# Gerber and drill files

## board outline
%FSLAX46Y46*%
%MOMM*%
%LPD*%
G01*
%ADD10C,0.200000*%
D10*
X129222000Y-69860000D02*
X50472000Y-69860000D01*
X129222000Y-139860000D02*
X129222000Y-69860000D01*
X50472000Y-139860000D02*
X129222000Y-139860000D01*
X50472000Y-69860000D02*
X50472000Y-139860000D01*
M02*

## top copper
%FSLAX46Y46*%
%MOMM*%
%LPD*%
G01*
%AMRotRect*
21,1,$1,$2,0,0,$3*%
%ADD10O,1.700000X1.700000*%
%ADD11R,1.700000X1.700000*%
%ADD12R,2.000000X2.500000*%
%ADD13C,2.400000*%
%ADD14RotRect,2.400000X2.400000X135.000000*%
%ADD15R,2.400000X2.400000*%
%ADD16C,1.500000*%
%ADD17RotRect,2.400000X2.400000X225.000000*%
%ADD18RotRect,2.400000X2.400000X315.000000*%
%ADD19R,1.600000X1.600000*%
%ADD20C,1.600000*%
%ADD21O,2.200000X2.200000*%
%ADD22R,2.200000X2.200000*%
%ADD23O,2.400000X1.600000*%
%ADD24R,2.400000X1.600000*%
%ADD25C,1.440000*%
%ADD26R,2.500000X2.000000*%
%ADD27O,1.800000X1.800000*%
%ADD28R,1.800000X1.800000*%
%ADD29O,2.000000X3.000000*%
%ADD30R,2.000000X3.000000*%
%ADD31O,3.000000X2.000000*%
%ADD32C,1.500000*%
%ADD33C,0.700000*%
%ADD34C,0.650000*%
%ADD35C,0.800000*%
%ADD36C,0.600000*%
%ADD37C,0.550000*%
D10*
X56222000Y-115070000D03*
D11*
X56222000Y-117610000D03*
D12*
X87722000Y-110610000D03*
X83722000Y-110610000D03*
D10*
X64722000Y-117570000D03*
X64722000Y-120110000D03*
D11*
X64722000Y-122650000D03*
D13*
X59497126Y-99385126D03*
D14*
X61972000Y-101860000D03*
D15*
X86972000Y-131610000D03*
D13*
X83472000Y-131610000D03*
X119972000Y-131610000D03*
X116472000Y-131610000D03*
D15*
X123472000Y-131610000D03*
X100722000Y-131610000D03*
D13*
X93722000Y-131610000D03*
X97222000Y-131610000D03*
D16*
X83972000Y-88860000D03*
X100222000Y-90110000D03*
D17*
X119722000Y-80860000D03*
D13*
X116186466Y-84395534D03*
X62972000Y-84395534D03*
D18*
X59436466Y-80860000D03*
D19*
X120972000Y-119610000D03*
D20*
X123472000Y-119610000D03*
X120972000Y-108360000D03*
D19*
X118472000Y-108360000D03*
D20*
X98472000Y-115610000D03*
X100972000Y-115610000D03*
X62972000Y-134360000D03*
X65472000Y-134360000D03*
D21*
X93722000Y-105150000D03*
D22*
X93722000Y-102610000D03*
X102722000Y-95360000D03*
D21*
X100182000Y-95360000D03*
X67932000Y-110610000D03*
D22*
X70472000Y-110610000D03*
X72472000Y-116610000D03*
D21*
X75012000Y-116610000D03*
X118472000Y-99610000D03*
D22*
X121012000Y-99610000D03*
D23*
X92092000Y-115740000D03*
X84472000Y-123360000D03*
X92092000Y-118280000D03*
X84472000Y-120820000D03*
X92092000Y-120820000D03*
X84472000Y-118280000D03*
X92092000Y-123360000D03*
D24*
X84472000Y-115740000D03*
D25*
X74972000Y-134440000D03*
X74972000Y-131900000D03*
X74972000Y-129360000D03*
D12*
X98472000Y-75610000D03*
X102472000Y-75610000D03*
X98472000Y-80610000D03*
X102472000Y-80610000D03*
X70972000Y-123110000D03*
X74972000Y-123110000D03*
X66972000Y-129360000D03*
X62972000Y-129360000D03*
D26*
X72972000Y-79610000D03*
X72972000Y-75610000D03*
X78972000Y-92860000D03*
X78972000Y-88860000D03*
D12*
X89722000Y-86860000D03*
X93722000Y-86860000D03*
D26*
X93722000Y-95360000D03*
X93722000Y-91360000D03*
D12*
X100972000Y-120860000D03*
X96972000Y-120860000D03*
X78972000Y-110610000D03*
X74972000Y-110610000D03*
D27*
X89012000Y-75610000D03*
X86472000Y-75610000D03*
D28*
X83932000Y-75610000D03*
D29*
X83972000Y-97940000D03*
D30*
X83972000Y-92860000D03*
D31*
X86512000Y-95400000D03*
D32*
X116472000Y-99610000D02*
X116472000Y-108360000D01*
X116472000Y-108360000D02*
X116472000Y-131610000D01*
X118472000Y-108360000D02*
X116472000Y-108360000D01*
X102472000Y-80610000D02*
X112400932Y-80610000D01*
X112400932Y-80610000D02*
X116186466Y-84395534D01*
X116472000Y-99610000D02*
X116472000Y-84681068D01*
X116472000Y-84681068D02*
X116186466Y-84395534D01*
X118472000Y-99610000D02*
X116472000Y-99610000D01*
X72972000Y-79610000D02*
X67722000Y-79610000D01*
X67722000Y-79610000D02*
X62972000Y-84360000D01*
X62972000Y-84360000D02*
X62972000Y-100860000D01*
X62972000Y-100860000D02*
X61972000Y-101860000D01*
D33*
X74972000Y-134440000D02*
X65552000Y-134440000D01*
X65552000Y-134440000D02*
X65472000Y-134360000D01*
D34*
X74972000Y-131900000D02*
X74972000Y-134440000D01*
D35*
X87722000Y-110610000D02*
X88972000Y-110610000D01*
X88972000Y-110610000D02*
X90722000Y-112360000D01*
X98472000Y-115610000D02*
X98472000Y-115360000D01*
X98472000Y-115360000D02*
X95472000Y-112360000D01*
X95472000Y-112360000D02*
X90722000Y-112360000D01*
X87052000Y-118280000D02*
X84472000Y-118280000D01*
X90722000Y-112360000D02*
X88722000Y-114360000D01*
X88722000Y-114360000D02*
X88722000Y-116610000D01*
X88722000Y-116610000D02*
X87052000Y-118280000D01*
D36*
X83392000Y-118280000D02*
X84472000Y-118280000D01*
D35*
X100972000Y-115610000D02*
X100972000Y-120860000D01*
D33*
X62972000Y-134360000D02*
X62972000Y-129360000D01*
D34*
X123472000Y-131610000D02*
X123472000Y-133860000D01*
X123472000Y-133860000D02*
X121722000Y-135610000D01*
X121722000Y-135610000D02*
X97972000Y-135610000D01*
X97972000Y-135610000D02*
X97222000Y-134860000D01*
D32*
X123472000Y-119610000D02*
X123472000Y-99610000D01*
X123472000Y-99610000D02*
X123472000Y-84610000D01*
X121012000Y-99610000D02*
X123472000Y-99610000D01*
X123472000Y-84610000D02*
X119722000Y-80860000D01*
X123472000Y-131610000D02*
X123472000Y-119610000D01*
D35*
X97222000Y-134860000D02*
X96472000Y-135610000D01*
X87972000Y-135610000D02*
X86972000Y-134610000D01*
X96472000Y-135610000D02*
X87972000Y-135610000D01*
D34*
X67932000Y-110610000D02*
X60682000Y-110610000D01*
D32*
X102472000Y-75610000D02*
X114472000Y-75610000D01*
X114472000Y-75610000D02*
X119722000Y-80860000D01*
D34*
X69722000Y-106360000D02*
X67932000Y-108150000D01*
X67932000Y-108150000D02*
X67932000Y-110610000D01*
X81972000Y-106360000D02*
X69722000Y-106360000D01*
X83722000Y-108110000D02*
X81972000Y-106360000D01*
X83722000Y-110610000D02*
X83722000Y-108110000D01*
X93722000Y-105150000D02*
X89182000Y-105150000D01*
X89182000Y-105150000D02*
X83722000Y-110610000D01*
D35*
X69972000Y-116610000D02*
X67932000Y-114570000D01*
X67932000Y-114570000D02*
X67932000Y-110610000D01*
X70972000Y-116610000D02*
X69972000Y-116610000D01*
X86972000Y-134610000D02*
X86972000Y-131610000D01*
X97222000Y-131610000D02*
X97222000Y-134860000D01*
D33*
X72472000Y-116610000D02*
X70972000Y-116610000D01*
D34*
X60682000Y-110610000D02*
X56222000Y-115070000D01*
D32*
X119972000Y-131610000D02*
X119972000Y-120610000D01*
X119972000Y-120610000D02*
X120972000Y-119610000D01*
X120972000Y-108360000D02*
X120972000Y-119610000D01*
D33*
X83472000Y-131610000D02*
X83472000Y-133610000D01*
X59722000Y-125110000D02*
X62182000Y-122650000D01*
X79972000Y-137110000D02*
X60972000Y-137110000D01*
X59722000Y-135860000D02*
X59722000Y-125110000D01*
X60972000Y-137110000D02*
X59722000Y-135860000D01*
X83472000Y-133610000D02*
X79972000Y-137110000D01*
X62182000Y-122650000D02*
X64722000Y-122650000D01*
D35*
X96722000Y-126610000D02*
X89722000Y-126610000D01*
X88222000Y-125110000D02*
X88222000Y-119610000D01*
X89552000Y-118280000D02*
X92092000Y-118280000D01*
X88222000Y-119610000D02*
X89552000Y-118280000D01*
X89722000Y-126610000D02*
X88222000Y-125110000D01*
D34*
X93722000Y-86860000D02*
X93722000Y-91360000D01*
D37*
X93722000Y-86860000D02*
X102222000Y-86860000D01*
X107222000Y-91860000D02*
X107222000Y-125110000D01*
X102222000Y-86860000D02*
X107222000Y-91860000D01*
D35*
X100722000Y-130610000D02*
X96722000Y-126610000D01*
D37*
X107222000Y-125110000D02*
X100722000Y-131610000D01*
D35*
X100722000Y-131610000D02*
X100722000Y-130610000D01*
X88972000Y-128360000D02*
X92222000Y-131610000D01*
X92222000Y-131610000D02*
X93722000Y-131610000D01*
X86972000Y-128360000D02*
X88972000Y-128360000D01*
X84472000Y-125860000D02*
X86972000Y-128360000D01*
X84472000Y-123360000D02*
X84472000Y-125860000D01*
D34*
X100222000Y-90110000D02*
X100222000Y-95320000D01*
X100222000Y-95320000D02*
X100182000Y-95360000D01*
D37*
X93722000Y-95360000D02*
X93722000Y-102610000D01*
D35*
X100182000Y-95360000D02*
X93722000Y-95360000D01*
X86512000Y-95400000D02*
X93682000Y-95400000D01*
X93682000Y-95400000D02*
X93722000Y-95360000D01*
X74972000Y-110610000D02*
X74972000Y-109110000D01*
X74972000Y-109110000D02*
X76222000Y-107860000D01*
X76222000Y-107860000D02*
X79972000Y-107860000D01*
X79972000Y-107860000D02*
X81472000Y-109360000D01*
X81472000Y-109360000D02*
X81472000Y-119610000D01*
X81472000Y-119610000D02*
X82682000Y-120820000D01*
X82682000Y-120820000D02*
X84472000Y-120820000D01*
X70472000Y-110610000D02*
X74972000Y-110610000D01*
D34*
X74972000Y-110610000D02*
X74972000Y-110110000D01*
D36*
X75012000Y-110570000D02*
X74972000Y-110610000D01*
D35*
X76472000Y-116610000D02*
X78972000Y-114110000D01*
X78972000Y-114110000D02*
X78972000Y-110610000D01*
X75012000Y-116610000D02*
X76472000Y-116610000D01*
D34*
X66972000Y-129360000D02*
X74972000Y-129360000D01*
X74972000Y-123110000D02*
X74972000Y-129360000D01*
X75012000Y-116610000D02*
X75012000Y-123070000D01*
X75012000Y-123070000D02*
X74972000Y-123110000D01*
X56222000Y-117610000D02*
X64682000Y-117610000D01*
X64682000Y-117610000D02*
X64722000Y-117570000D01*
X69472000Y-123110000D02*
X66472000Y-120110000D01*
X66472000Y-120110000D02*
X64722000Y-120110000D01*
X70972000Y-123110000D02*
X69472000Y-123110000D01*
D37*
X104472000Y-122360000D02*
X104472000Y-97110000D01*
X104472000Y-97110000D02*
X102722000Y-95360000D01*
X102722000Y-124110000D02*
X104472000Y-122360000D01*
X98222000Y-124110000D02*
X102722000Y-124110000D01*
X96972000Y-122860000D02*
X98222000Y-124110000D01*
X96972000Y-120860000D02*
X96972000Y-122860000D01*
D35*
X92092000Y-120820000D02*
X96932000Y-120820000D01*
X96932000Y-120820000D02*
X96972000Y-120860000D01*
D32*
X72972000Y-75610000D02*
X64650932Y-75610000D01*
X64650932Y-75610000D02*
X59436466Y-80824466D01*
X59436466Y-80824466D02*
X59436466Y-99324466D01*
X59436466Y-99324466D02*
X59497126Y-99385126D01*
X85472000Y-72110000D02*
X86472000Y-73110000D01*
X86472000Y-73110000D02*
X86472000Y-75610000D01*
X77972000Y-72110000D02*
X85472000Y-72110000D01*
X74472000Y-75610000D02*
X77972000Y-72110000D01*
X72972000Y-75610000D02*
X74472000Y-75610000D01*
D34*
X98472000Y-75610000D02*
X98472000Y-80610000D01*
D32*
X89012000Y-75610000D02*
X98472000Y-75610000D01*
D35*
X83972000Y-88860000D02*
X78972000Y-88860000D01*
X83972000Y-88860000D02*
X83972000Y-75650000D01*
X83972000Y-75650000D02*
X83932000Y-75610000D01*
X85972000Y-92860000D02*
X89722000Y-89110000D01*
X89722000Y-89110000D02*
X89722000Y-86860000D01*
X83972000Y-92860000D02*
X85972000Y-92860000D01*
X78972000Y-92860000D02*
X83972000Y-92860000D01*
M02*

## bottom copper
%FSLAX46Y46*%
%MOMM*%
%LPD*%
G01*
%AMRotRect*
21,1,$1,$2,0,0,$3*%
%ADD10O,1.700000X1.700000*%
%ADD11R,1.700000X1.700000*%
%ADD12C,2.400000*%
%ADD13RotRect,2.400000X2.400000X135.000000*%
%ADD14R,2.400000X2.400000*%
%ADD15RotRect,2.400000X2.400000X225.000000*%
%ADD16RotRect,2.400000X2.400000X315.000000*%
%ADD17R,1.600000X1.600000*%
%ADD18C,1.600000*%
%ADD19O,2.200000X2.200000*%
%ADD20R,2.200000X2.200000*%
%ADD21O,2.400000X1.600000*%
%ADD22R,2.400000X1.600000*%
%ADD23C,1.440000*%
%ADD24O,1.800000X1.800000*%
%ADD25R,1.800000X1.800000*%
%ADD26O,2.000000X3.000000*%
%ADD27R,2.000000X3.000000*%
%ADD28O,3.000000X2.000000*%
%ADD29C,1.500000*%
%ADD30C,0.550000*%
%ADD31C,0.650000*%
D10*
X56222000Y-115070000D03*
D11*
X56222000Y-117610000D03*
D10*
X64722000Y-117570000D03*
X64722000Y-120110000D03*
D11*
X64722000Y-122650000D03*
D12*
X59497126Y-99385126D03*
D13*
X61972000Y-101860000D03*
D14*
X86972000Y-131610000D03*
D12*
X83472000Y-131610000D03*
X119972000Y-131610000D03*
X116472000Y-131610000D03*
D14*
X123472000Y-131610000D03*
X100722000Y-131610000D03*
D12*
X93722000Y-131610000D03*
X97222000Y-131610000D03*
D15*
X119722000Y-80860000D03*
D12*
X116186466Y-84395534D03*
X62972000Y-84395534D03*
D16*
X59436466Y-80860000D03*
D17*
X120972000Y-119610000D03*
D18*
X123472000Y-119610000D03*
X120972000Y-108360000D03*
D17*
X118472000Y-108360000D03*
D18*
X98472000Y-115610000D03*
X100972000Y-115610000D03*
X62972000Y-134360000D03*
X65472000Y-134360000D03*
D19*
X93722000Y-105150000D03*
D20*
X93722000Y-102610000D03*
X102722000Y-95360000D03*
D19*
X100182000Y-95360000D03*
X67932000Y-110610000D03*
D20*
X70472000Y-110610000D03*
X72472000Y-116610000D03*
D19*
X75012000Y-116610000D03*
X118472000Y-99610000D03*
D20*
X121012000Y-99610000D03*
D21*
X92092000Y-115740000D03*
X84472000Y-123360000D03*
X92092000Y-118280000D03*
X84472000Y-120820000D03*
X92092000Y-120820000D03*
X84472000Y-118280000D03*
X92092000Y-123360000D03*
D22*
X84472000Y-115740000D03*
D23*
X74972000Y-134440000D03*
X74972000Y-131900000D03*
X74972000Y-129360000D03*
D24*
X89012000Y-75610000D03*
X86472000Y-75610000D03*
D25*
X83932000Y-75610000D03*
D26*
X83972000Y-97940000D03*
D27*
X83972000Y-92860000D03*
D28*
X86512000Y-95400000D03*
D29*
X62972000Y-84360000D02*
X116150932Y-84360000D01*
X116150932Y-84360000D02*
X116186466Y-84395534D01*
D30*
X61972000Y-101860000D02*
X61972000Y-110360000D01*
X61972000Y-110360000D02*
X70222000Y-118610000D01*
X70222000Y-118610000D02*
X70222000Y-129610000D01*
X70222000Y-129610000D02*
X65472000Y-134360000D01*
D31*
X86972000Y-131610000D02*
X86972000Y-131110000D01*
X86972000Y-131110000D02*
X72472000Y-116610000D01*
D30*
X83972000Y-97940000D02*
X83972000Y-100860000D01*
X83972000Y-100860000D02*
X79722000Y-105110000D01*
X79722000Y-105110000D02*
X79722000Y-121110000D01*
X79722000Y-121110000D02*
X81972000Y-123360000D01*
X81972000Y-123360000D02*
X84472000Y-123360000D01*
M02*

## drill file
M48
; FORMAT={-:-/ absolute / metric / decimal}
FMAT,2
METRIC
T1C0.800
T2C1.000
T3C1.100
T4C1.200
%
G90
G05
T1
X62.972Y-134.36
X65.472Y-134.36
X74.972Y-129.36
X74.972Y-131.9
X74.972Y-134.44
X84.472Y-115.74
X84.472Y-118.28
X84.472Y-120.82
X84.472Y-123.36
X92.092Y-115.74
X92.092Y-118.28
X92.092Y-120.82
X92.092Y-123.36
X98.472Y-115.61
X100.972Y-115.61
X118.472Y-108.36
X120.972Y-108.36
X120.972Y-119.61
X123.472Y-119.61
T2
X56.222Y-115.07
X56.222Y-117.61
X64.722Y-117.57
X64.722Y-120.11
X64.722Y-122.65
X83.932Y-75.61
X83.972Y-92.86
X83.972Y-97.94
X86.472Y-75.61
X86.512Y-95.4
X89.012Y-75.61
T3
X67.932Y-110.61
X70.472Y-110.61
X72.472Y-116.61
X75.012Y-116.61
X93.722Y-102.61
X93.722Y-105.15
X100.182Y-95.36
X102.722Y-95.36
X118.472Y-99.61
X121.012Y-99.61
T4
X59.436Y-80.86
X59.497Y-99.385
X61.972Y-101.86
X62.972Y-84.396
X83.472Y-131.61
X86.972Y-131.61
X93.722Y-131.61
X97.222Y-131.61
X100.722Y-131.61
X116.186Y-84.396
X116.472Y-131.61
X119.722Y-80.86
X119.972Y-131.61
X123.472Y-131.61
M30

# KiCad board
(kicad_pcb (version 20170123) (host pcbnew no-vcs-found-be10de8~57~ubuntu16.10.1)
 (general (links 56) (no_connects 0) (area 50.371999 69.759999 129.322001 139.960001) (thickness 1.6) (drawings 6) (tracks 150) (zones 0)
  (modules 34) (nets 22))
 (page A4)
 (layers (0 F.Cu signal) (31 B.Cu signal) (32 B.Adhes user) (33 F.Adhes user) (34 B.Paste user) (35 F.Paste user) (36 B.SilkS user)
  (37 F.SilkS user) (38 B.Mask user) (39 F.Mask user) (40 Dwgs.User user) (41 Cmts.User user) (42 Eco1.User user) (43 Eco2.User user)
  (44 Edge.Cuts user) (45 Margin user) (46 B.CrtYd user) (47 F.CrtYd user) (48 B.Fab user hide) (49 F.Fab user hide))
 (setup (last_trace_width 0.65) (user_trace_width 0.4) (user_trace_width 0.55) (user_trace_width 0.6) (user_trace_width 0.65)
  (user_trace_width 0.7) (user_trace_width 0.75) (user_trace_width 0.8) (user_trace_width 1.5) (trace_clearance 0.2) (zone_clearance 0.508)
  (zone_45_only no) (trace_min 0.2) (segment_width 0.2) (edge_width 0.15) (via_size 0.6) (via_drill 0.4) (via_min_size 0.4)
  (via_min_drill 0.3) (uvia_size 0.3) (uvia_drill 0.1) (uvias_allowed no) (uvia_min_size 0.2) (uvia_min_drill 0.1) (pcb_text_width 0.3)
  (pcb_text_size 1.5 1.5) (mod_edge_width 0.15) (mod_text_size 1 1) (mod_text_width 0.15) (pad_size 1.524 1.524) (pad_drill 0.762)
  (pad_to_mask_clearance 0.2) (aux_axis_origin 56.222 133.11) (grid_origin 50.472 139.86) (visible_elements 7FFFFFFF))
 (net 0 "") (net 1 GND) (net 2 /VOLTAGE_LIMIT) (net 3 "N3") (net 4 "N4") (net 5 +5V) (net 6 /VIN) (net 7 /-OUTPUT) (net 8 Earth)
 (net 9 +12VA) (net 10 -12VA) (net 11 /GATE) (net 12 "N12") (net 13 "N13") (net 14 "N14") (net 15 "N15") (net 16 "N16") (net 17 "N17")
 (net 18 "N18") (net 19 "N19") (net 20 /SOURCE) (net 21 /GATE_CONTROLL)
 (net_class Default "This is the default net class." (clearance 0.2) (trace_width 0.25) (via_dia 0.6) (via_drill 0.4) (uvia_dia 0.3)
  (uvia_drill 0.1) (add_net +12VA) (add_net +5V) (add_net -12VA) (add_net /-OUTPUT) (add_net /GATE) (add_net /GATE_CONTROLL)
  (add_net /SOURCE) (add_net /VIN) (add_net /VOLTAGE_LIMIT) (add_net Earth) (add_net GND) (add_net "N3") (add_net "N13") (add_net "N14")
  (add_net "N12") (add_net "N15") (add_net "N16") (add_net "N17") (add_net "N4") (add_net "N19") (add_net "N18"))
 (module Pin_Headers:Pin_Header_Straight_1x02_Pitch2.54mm (layer F.Cu) (at 56.222 117.61 180)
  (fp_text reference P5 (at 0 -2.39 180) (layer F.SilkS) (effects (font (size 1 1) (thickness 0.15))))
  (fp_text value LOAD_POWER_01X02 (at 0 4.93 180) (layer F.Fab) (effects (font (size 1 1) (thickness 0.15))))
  (pad 2 thru_hole oval (at 0 2.54 180) (size 1.7 1.7) (drill 1) (layers *.Cu *.Mask) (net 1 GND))
  (pad 1 thru_hole rect (at 0 0 180) (size 1.7 1.7) (drill 1) (layers *.Cu *.Mask) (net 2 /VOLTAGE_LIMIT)))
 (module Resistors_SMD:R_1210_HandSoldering (layer F.Cu) (at 85.722 110.61 180)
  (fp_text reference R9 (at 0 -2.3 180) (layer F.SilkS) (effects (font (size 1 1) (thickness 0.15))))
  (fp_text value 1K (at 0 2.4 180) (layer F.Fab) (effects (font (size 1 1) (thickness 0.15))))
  (pad 1 smd rect (at -2 0 180) (size 2 2.5) (layers F.Cu F.Paste F.Mask) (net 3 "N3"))
  (pad 2 smd rect (at 2 0 180) (size 2 2.5) (layers F.Cu F.Paste F.Mask) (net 1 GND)))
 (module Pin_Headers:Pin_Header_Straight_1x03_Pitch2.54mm (layer F.Cu) (at 64.722 122.65 180)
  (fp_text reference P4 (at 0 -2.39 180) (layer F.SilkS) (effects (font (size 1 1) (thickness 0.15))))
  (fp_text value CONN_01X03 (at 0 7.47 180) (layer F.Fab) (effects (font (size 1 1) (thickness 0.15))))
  (pad 3 thru_hole oval (at 0 5.08 180) (size 1.7 1.7) (drill 1) (layers *.Cu *.Mask) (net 2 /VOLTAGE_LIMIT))
  (pad 2 thru_hole oval (at 0 2.54 180) (size 1.7 1.7) (drill 1) (layers *.Cu *.Mask) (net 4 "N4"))
  (pad 1 thru_hole rect (at 0 0 180) (size 1.7 1.7) (drill 1) (layers *.Cu *.Mask) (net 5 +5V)))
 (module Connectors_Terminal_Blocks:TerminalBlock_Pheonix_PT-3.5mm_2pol (layer B.Cu) (at 61.972 101.86 135)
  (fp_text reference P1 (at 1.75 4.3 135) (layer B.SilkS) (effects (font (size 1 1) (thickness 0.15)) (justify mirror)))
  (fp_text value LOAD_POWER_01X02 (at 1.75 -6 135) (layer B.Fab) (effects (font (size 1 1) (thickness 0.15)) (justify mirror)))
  (pad 2 thru_hole circle (at 3.5 0 135) (size 2.4 2.4) (drill 1.2) (layers *.Cu *.Mask) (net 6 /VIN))
  (pad 1 thru_hole rect (at 0 0 135) (size 2.4 2.4) (drill 1.2) (layers *.Cu *.Mask) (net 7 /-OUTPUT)))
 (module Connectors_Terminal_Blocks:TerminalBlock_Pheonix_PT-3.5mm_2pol (layer B.Cu) (at 86.972 131.61 180)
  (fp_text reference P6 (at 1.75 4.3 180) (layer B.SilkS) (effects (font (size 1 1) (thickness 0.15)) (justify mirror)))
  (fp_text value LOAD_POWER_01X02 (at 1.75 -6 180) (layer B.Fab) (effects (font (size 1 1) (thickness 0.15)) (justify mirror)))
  (pad 1 thru_hole rect (at 0 0 180) (size 2.4 2.4) (drill 1.2) (layers *.Cu *.Mask) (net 1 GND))
  (pad 2 thru_hole circle (at 3.5 0 180) (size 2.4 2.4) (drill 1.2) (layers *.Cu *.Mask) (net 5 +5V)))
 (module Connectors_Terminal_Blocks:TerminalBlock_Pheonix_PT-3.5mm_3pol (layer B.Cu) (at 123.472 131.61 180)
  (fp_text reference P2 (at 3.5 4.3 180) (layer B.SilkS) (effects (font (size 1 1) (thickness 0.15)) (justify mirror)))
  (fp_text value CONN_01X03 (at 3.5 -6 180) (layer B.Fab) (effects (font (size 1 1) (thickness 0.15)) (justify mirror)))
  (pad 2 thru_hole circle (at 3.5 0 180) (size 2.4 2.4) (drill 1.2) (layers *.Cu *.Mask) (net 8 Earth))
  (pad 3 thru_hole circle (at 7 0 180) (size 2.4 2.4) (drill 1.2) (layers *.Cu *.Mask) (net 7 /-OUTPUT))
  (pad 1 thru_hole rect (at 0 0 180) (size 2.4 2.4) (drill 1.2) (layers *.Cu *.Mask) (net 1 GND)))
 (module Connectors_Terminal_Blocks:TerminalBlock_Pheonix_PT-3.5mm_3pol (layer B.Cu) (at 100.722 131.61 180)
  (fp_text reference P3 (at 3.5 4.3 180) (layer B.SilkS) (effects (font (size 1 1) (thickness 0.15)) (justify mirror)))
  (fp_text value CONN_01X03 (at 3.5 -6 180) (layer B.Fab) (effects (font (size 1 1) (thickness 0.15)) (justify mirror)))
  (pad 1 thru_hole rect (at 0 0 180) (size 2.4 2.4) (drill 1.2) (layers *.Cu *.Mask) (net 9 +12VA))
  (pad 3 thru_hole circle (at 7 0 180) (size 2.4 2.4) (drill 1.2) (layers *.Cu *.Mask) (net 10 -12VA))
  (pad 2 thru_hole circle (at 3.5 0 180) (size 2.4 2.4) (drill 1.2) (layers *.Cu *.Mask) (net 1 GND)))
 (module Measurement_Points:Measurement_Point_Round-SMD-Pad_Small (layer F.Cu) (at 83.972 88.86)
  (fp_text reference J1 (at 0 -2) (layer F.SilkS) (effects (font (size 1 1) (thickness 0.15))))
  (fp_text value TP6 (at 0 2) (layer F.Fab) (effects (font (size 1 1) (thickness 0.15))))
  (pad 1 smd circle (at 0 0) (size 1.5 1.5) (layers F.Cu F.Mask) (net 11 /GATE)))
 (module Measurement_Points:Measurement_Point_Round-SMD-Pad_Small (layer F.Cu) (at 100.222 90.11)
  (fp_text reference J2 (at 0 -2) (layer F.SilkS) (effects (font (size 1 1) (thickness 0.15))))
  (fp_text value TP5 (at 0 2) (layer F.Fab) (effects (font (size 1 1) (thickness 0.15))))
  (pad 1 smd circle (at 0 0) (size 1.5 1.5) (layers F.Cu F.Mask) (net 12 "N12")))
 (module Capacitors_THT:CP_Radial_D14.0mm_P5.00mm (layer B.Cu) (at 119.722 80.86 225)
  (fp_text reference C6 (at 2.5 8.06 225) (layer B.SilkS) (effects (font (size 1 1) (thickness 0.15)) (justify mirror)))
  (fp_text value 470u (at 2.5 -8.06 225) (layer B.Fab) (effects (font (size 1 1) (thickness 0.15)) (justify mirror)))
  (pad 1 thru_hole rect (at 0 0 225) (size 2.4 2.4) (drill 1.2) (layers *.Cu *.Mask) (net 1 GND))
  (pad 2 thru_hole circle (at 5 0 225) (size 2.4 2.4) (drill 1.2) (layers *.Cu *.Mask) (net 7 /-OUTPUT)))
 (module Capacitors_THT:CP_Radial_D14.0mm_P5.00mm (layer B.Cu) (at 59.436466 80.86 315)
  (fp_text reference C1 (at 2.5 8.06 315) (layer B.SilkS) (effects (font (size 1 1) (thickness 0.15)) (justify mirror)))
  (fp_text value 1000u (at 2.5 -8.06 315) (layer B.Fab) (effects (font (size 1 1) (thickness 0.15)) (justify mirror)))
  (pad 2 thru_hole circle (at 5 0 315) (size 2.4 2.4) (drill 1.2) (layers *.Cu *.Mask) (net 7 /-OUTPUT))
  (pad 1 thru_hole rect (at 0 0 315) (size 2.4 2.4) (drill 1.2) (layers *.Cu *.Mask) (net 6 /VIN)))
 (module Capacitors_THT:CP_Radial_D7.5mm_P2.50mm (layer B.Cu) (at 120.972 119.61)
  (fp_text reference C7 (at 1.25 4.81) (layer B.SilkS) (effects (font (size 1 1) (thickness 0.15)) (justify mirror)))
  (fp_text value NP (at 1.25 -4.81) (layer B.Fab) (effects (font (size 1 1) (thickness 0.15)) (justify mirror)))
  (pad 1 thru_hole rect (at 0 0) (size 1.6 1.6) (drill 0.8) (layers *.Cu *.Mask) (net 8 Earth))
  (pad 2 thru_hole circle (at 2.5 0) (size 1.6 1.6) (drill 0.8) (layers *.Cu *.Mask) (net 1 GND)))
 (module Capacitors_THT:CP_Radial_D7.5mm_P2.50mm (layer B.Cu) (at 118.472 108.36)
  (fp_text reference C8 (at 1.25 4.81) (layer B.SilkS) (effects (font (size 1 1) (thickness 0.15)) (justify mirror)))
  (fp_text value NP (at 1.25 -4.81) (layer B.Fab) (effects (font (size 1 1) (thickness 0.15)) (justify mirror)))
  (pad 2 thru_hole circle (at 2.5 0) (size 1.6 1.6) (drill 0.8) (layers *.Cu *.Mask) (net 8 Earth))
  (pad 1 thru_hole rect (at 0 0) (size 1.6 1.6) (drill 0.8) (layers *.Cu *.Mask) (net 7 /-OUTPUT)))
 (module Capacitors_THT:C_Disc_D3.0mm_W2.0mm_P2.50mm (layer F.Cu) (at 98.472 115.61)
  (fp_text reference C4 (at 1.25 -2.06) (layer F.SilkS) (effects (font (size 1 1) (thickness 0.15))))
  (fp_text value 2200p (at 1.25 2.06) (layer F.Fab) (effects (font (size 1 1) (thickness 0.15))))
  (pad 1 thru_hole circle (at 0 0) (size 1.6 1.6) (drill 0.8) (layers *.Cu *.Mask) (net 3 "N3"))
  (pad 2 thru_hole circle (at 2.5 0) (size 1.6 1.6) (drill 0.8) (layers *.Cu *.Mask) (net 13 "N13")))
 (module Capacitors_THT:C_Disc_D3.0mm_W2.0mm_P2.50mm (layer F.Cu) (at 65.472 134.36 180)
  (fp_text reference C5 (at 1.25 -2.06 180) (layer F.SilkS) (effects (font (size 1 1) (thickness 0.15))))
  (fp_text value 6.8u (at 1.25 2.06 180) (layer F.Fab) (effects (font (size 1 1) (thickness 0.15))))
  (pad 2 thru_hole circle (at 2.5 0 180) (size 1.6 1.6) (drill 0.8) (layers *.Cu *.Mask) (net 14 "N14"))
  (pad 1 thru_hole circle (at 0 0 180) (size 1.6 1.6) (drill 0.8) (layers *.Cu *.Mask) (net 7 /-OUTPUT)))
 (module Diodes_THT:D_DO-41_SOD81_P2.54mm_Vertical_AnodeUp (layer F.Cu) (at 93.722 102.61 270)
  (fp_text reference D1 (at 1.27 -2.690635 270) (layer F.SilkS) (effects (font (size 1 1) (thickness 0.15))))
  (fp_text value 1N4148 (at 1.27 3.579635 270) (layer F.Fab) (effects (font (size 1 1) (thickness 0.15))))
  (pad 2 thru_hole oval (at 2.54 0 270) (size 2.2 2.2) (drill 1.1) (layers *.Cu *.Mask) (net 1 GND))
  (pad 1 thru_hole rect (at 0 0 270) (size 2.2 2.2) (drill 1.1) (layers *.Cu *.Mask) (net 12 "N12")))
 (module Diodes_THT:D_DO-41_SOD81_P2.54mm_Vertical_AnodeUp (layer F.Cu) (at 102.722 95.36 180)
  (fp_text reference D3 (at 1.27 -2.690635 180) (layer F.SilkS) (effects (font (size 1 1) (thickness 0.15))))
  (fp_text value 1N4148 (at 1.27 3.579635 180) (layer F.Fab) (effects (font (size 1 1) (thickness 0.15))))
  (pad 1 thru_hole rect (at 0 0 180) (size 2.2 2.2) (drill 1.1) (layers *.Cu *.Mask) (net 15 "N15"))
  (pad 2 thru_hole oval (at 2.54 0 180) (size 2.2 2.2) (drill 1.1) (layers *.Cu *.Mask) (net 12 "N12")))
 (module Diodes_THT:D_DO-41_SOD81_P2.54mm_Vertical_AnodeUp (layer F.Cu) (at 70.472 110.61 180)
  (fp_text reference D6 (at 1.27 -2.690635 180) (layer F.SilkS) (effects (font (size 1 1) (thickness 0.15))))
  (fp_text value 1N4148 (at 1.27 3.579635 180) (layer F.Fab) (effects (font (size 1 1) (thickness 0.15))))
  (pad 2 thru_hole oval (at 2.54 0 180) (size 2.2 2.2) (drill 1.1) (layers *.Cu *.Mask) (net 1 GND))
  (pad 1 thru_hole rect (at 0 0 180) (size 2.2 2.2) (drill 1.1) (layers *.Cu *.Mask) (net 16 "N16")))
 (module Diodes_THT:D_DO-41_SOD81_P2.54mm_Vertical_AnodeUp (layer F.Cu) (at 72.472 116.61)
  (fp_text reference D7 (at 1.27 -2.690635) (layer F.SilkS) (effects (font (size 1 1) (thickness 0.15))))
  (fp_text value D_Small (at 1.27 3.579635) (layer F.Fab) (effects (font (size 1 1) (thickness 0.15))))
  (pad 1 thru_hole rect (at 0 0) (size 2.2 2.2) (drill 1.1) (layers *.Cu *.Mask) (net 1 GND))
  (pad 2 thru_hole oval (at 2.54 0) (size 2.2 2.2) (drill 1.1) (layers *.Cu *.Mask) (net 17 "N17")))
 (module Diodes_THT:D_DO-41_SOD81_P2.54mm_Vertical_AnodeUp (layer F.Cu) (at 121.012 99.61 180)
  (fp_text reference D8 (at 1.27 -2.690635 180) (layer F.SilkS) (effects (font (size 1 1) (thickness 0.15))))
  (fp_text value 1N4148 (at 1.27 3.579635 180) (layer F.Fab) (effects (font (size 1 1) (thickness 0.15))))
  (pad 2 thru_hole oval (at 2.54 0 180) (size 2.2 2.2) (drill 1.1) (layers *.Cu *.Mask) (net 7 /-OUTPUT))
  (pad 1 thru_hole rect (at 0 0 180) (size 2.2 2.2) (drill 1.1) (layers *.Cu *.Mask) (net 1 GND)))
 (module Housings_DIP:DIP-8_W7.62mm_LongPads (layer F.Cu) (at 84.472 115.74)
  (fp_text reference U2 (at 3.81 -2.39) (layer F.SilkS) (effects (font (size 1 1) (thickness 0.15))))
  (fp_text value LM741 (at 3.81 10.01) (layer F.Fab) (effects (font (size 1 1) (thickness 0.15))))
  (pad 8 thru_hole oval (at 7.62 0) (size 2.4 1.6) (drill 0.8) (layers *.Cu *.Mask))
  (pad 4 thru_hole oval (at 0 7.62) (size 2.4 1.6) (drill 0.8) (layers *.Cu *.Mask) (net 10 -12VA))
  (pad 7 thru_hole oval (at 7.62 2.54) (size 2.4 1.6) (drill 0.8) (layers *.Cu *.Mask) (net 9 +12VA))
  (pad 3 thru_hole oval (at 0 5.08) (size 2.4 1.6) (drill 0.8) (layers *.Cu *.Mask) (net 16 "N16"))
  (pad 6 thru_hole oval (at 7.62 5.08) (size 2.4 1.6) (drill 0.8) (layers *.Cu *.Mask) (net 15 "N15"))
  (pad 2 thru_hole oval (at 0 2.54) (size 2.4 1.6) (drill 0.8) (layers *.Cu *.Mask) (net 3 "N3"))
  (pad 5 thru_hole oval (at 7.62 7.62) (size 2.4 1.6) (drill 0.8) (layers *.Cu *.Mask) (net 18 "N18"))
  (pad 1 thru_hole rect (at 0 0) (size 2.4 1.6) (drill 0.8) (layers *.Cu *.Mask) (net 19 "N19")))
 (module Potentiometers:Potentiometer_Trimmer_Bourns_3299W (layer F.Cu) (at 74.972 129.36 90)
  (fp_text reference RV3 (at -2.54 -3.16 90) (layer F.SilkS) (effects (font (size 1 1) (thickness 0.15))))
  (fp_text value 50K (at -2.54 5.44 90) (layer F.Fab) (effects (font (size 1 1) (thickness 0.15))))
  (pad 3 thru_hole circle (at -5.08 0 90) (size 1.44 1.44) (drill 0.8) (layers *.Cu *.Mask) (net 7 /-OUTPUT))
  (pad 2 thru_hole circle (at -2.54 0 90) (size 1.44 1.44) (drill 0.8) (layers *.Cu *.Mask) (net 7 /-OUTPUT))
  (pad 1 thru_hole circle (at 0 0 90) (size 1.44 1.44) (drill 0.8) (layers *.Cu *.Mask) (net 17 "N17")))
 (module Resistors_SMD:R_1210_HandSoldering (layer F.Cu) (at 100.472 75.61)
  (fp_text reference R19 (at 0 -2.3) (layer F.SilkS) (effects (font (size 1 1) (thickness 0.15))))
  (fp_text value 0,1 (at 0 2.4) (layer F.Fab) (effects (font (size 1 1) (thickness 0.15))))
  (pad 1 smd rect (at -2 0) (size 2 2.5) (layers F.Cu F.Paste F.Mask) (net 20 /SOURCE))
  (pad 2 smd rect (at 2 0) (size 2 2.5) (layers F.Cu F.Paste F.Mask) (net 1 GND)))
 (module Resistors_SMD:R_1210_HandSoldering (layer F.Cu) (at 100.472 80.61 180)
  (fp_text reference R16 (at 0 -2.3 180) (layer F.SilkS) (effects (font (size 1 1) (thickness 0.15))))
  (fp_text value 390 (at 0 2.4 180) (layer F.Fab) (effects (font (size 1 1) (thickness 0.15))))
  (pad 2 smd rect (at 2 0 180) (size 2 2.5) (layers F.Cu F.Paste F.Mask) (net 20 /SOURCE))
  (pad 1 smd rect (at -2 0 180) (size 2 2.5) (layers F.Cu F.Paste F.Mask) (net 7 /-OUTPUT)))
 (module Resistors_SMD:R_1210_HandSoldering (layer F.Cu) (at 72.972 123.11)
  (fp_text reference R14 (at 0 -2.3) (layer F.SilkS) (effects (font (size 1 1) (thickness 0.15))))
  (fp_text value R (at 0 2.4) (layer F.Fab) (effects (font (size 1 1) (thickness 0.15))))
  (pad 1 smd rect (at -2 0) (size 2 2.5) (layers F.Cu F.Paste F.Mask) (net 4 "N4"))
  (pad 2 smd rect (at 2 0) (size 2 2.5) (layers F.Cu F.Paste F.Mask) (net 17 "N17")))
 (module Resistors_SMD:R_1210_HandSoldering (layer F.Cu) (at 64.972 129.36)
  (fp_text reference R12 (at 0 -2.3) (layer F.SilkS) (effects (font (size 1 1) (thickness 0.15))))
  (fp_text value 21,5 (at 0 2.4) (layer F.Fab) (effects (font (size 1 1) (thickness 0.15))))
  (pad 2 smd rect (at 2 0) (size 2 2.5) (layers F.Cu F.Paste F.Mask) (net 17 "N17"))
  (pad 1 smd rect (at -2 0) (size 2 2.5) (layers F.Cu F.Paste F.Mask) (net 14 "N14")))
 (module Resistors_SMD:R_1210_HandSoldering (layer F.Cu) (at 72.972 77.61 270)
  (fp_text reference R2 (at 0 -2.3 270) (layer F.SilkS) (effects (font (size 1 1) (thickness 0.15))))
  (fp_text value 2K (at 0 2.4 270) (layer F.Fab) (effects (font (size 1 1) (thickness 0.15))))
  (pad 2 smd rect (at 2 0 270) (size 2 2.5) (layers F.Cu F.Paste F.Mask) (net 7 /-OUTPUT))
  (pad 1 smd rect (at -2 0 270) (size 2 2.5) (layers F.Cu F.Paste F.Mask) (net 6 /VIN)))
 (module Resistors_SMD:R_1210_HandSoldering (layer F.Cu) (at 78.972 90.86 90)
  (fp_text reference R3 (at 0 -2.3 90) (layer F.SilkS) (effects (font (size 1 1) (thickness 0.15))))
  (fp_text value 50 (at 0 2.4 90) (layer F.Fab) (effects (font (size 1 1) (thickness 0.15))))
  (pad 1 smd rect (at -2 0 90) (size 2 2.5) (layers F.Cu F.Paste F.Mask) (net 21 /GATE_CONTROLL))
  (pad 2 smd rect (at 2 0 90) (size 2 2.5) (layers F.Cu F.Paste F.Mask) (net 11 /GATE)))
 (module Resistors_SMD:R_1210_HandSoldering (layer F.Cu) (at 91.722 86.86 180)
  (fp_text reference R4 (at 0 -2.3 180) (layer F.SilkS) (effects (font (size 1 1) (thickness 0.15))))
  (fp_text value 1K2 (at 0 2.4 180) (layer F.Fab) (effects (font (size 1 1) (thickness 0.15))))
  (pad 2 smd rect (at 2 0 180) (size 2 2.5) (layers F.Cu F.Paste F.Mask) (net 21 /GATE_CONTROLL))
  (pad 1 smd rect (at -2 0 180) (size 2 2.5) (layers F.Cu F.Paste F.Mask) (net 9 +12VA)))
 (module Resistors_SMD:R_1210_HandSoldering (layer F.Cu) (at 93.722 93.36 90)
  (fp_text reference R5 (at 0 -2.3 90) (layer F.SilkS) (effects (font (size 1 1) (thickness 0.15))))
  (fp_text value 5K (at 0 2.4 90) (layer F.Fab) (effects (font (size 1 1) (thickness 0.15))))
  (pad 1 smd rect (at -2 0 90) (size 2 2.5) (layers F.Cu F.Paste F.Mask) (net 12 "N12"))
  (pad 2 smd rect (at 2 0 90) (size 2 2.5) (layers F.Cu F.Paste F.Mask) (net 9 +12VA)))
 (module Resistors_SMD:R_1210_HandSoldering (layer F.Cu) (at 98.972 120.86)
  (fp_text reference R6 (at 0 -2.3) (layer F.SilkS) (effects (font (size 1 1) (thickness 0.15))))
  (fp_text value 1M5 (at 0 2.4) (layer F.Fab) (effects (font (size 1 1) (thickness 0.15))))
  (pad 2 smd rect (at 2 0) (size 2 2.5) (layers F.Cu F.Paste F.Mask) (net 13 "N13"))
  (pad 1 smd rect (at -2 0) (size 2 2.5) (layers F.Cu F.Paste F.Mask) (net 15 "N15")))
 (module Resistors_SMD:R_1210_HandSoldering (layer F.Cu) (at 76.972 110.61)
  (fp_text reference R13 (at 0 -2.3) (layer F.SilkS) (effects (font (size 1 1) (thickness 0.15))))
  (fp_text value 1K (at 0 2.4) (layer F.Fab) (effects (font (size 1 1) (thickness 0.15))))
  (pad 2 smd rect (at 2 0) (size 2 2.5) (layers F.Cu F.Paste F.Mask) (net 17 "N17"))
  (pad 1 smd rect (at -2 0) (size 2 2.5) (layers F.Cu F.Paste F.Mask) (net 16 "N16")))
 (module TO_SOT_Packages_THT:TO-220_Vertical (layer F.Cu) (at 83.932 75.61)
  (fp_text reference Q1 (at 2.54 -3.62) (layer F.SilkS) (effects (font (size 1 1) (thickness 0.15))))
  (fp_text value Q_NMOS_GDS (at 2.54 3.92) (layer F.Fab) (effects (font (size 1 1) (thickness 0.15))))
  (pad 3 thru_hole oval (at 5.08 0) (size 1.8 1.8) (drill 1) (layers *.Cu *.Mask) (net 20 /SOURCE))
  (pad 2 thru_hole oval (at 2.54 0) (size 1.8 1.8) (drill 1) (layers *.Cu *.Mask) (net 6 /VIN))
  (pad 1 thru_hole rect (at 0 0) (size 1.8 1.8) (drill 1) (layers *.Cu *.Mask) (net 11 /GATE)))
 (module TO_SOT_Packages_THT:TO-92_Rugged (layer F.Cu) (at 83.972 92.86 270)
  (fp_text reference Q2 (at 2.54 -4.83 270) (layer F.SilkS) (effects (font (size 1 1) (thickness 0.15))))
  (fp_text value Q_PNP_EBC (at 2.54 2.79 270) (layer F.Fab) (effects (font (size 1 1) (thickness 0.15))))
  (pad 3 thru_hole oval (at 5.08 0) (size 2 3) (drill 1) (layers *.Cu *.Mask) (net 10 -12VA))
  (pad 1 thru_hole rect (at 0 0) (size 2 3) (drill 1) (layers *.Cu *.Mask) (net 21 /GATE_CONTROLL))
  (pad 2 thru_hole oval (at 2.54 -2.54) (size 3 2) (drill 1) (layers *.Cu *.Mask) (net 12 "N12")))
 (gr_line (start 129.222 69.86) (end 50.472 69.86) (layer Edge.Cuts) (width 0.2))
 (gr_line (start 129.222 139.86) (end 129.222 69.86) (layer Edge.Cuts) (width 0.2))
 (gr_line (start 50.472 139.86) (end 129.222 139.86) (layer Edge.Cuts) (width 0.2))
 (gr_line (start 50.472 69.86) (end 50.472 139.86) (layer Edge.Cuts) (width 0.2))
 (segment (start 116.472 99.61) (end 116.472 108.36) (width 1.5) (layer F.Cu) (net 7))
 (segment (start 116.472 108.36) (end 116.472 131.61) (width 1.5) (layer F.Cu) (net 7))
 (segment (start 118.472 108.36) (end 116.472 108.36) (width 1.5) (layer F.Cu) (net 7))
 (segment (start 102.472 80.61) (end 112.400932 80.61) (width 1.5) (layer F.Cu) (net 7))
 (segment (start 112.400932 80.61) (end 116.186466 84.395534) (width 1.5) (layer F.Cu) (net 7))
 (segment (start 116.472 99.61) (end 116.472 84.681068) (width 1.5) (layer F.Cu) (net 7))
 (segment (start 116.472 84.681068) (end 116.186466 84.395534) (width 1.5) (layer F.Cu) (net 7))
 (segment (start 62.972 84.36) (end 116.150932 84.36) (width 1.5) (layer B.Cu) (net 7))
 (segment (start 116.150932 84.36) (end 116.186466 84.395534) (width 1.5) (layer B.Cu) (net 7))
 (segment (start 61.972 101.86) (end 61.972 110.36) (width 0.55) (layer B.Cu) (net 7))
 (segment (start 61.972 110.36) (end 70.222 118.61) (width 0.55) (layer B.Cu) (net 7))
 (segment (start 70.222 118.61) (end 70.222 129.61) (width 0.55) (layer B.Cu) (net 7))
 (segment (start 70.222 129.61) (end 65.472 134.36) (width 0.55) (layer B.Cu) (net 7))
 (segment (start 118.472 99.61) (end 116.472 99.61) (width 1.5) (layer F.Cu) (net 7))
 (segment (start 72.972 79.61) (end 67.722 79.61) (width 1.5) (layer F.Cu) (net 7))
 (segment (start 67.722 79.61) (end 62.972 84.36) (width 1.5) (layer F.Cu) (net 7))
 (segment (start 62.972 84.36) (end 62.972 100.86) (width 1.5) (layer F.Cu) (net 7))
 (segment (start 62.972 100.86) (end 61.972 101.86) (width 1.5) (layer F.Cu) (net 7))
 (segment (start 74.972 134.44) (end 65.552 134.44) (width 0.7) (layer F.Cu) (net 7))
 (segment (start 65.552 134.44) (end 65.472 134.36) (width 0.7) (layer F.Cu) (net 7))
 (segment (start 74.972 131.9) (end 74.972 134.44) (width 0.65) (layer F.Cu) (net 7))
 (segment (start 87.722 110.61) (end 88.972 110.61) (width 0.8) (layer F.Cu) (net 3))
 (segment (start 88.972 110.61) (end 90.722 112.36) (width 0.8) (layer F.Cu) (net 3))
 (segment (start 98.472 115.61) (end 98.472 115.36) (width 0.8) (layer F.Cu) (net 3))
 (segment (start 98.472 115.36) (end 95.472 112.36) (width 0.8) (layer F.Cu) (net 3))
 (segment (start 95.472 112.36) (end 90.722 112.36) (width 0.8) (layer F.Cu) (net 3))
 (segment (start 87.052 118.28) (end 84.472 118.28) (width 0.8) (layer F.Cu) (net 3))
 (segment (start 90.722 112.36) (end 88.722 114.36) (width 0.8) (layer F.Cu) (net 3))
 (segment (start 88.722 114.36) (end 88.722 116.61) (width 0.8) (layer F.Cu) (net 3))
 (segment (start 88.722 116.61) (end 87.052 118.28) (width 0.8) (layer F.Cu) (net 3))
 (segment (start 83.392 118.28) (end 84.472 118.28) (width 0.6) (layer F.Cu) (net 3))
 (segment (start 100.972 115.61) (end 100.972 120.86) (width 0.8) (layer F.Cu) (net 13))
 (segment (start 62.972 134.36) (end 62.972 129.36) (width 0.7) (layer F.Cu) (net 14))
 (segment (start 123.472 131.61) (end 123.472 133.86) (width 0.65) (layer F.Cu) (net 1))
 (segment (start 123.472 133.86) (end 121.722 135.61) (width 0.65) (layer F.Cu) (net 1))
 (segment (start 121.722 135.61) (end 97.972 135.61) (width 0.65) (layer F.Cu) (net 1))
 (segment (start 97.972 135.61) (end 97.222 134.86) (width 0.65) (layer F.Cu) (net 1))
 (segment (start 123.472 119.61) (end 123.472 99.61) (width 1.5) (layer F.Cu) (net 1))
 (segment (start 123.472 99.61) (end 123.472 84.61) (width 1.5) (layer F.Cu) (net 1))
 (segment (start 121.012 99.61) (end 123.472 99.61) (width 1.5) (layer F.Cu) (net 1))
 (segment (start 123.472 84.61) (end 119.722 80.86) (width 1.5) (layer F.Cu) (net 1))
 (segment (start 123.472 131.61) (end 123.472 119.61) (width 1.5) (layer F.Cu) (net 1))
 (segment (start 97.222 134.86) (end 96.472 135.61) (width 0.8) (layer F.Cu) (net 1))
 (segment (start 87.972 135.61) (end 86.972 134.61) (width 0.8) (layer F.Cu) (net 1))
 (segment (start 96.472 135.61) (end 87.972 135.61) (width 0.8) (layer F.Cu) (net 1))
 (segment (start 67.932 110.61) (end 60.682 110.61) (width 0.65) (layer F.Cu) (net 1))
 (segment (start 86.972 131.61) (end 86.972 131.11) (width 0.65) (layer B.Cu) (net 1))
 (segment (start 86.972 131.11) (end 72.472 116.61) (width 0.65) (layer B.Cu) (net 1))
 (segment (start 102.472 75.61) (end 114.472 75.61) (width 1.5) (layer F.Cu) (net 1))
 (segment (start 114.472 75.61) (end 119.722 80.86) (width 1.5) (layer F.Cu) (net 1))
 (segment (start 69.722 106.36) (end 67.932 108.15) (width 0.65) (layer F.Cu) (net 1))
 (segment (start 67.932 108.15) (end 67.932 110.61) (width 0.65) (layer F.Cu) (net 1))
 (segment (start 81.972 106.36) (end 69.722 106.36) (width 0.65) (layer F.Cu) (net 1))
 (segment (start 83.722 108.11) (end 81.972 106.36) (width 0.65) (layer F.Cu) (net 1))
 (segment (start 83.722 110.61) (end 83.722 108.11) (width 0.65) (layer F.Cu) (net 1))
 (segment (start 93.722 105.15) (end 89.182 105.15) (width 0.65) (layer F.Cu) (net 1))
 (segment (start 89.182 105.15) (end 83.722 110.61) (width 0.65) (layer F.Cu) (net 1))
 (segment (start 69.972 116.61) (end 67.932 114.57) (width 0.8) (layer F.Cu) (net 1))
 (segment (start 67.932 114.57) (end 67.932 110.61) (width 0.8) (layer F.Cu) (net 1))
 (segment (start 70.972 116.61) (end 69.972 116.61) (width 0.8) (layer F.Cu) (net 1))
 (segment (start 86.972 134.61) (end 86.972 131.61) (width 0.8) (layer F.Cu) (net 1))
 (segment (start 97.222 131.61) (end 97.222 134.86) (width 0.8) (layer F.Cu) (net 1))
 (segment (start 72.472 116.61) (end 70.972 116.61) (width 0.7) (layer F.Cu) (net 1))
 (segment (start 60.682 110.61) (end 56.222 115.07) (width 0.65) (layer F.Cu) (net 1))
 (segment (start 119.972 131.61) (end 119.972 120.61) (width 1.5) (layer F.Cu) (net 8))
 (segment (start 119.972 120.61) (end 120.972 119.61) (width 1.5) (layer F.Cu) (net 8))
 (segment (start 120.972 108.36) (end 120.972 119.61) (width 1.5) (layer F.Cu) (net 8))
 (segment (start 83.472 131.61) (end 83.472 133.61) (width 0.7) (layer F.Cu) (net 5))
 (segment (start 59.722 125.11) (end 62.182 122.65) (width 0.7) (layer F.Cu) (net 5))
 (segment (start 79.972 137.11) (end 60.972 137.11) (width 0.7) (layer F.Cu) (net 5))
 (segment (start 59.722 135.86) (end 59.722 125.11) (width 0.7) (layer F.Cu) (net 5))
 (segment (start 60.972 137.11) (end 59.722 135.86) (width 0.7) (layer F.Cu) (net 5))
 (segment (start 83.472 133.61) (end 79.972 137.11) (width 0.7) (layer F.Cu) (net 5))
 (segment (start 62.182 122.65) (end 64.722 122.65) (width 0.7) (layer F.Cu) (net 5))
 (segment (start 96.722 126.61) (end 89.722 126.61) (width 0.8) (layer F.Cu) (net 9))
 (segment (start 88.222 125.11) (end 88.222 119.61) (width 0.8) (layer F.Cu) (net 9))
 (segment (start 89.552 118.28) (end 92.092 118.28) (width 0.8) (layer F.Cu) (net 9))
 (segment (start 88.222 119.61) (end 89.552 118.28) (width 0.8) (layer F.Cu) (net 9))
 (segment (start 89.722 126.61) (end 88.222 125.11) (width 0.8) (layer F.Cu) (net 9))
 (segment (start 93.722 86.86) (end 93.722 91.36) (width 0.65) (layer F.Cu) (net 9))
 (segment (start 93.722 86.86) (end 102.222 86.86) (width 0.55) (layer F.Cu) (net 9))
 (segment (start 107.222 91.86) (end 107.222 125.11) (width 0.55) (layer F.Cu) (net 9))
 (segment (start 102.222 86.86) (end 107.222 91.86) (width 0.55) (layer F.Cu) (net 9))
 (segment (start 100.722 130.61) (end 96.722 126.61) (width 0.8) (layer F.Cu) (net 9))
 (segment (start 107.222 125.11) (end 100.722 131.61) (width 0.55) (layer F.Cu) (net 9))
 (segment (start 100.722 131.61) (end 100.722 130.61) (width 0.8) (layer F.Cu) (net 9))
 (segment (start 88.972 128.36) (end 92.222 131.61) (width 0.8) (layer F.Cu) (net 10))
 (segment (start 92.222 131.61) (end 93.722 131.61) (width 0.8) (layer F.Cu) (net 10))
 (segment (start 86.972 128.36) (end 88.972 128.36) (width 0.8) (layer F.Cu) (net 10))
 (segment (start 84.472 125.86) (end 86.972 128.36) (width 0.8) (layer F.Cu) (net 10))
 (segment (start 84.472 123.36) (end 84.472 125.86) (width 0.8) (layer F.Cu) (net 10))
 (segment (start 83.972 97.94) (end 83.972 100.86) (width 0.55) (layer B.Cu) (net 10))
 (segment (start 83.972 100.86) (end 79.722 105.11) (width 0.55) (layer B.Cu) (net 10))
 (segment (start 79.722 105.11) (end 79.722 121.11) (width 0.55) (layer B.Cu) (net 10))
 (segment (start 79.722 121.11) (end 81.972 123.36) (width 0.55) (layer B.Cu) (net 10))
 (segment (start 81.972 123.36) (end 84.472 123.36) (width 0.55) (layer B.Cu) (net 10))
 (segment (start 100.222 90.11) (end 100.222 95.32) (width 0.65) (layer F.Cu) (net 12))
 (segment (start 100.222 95.32) (end 100.182 95.36) (width 0.65) (layer F.Cu) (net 12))
 (segment (start 93.722 95.36) (end 93.722 102.61) (width 0.55) (layer F.Cu) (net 12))
 (segment (start 100.182 95.36) (end 93.722 95.36) (width 0.8) (layer F.Cu) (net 12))
 (segment (start 86.512 95.4) (end 93.682 95.4) (width 0.8) (layer F.Cu) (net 12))
 (segment (start 93.682 95.4) (end 93.722 95.36) (width 0.8) (layer F.Cu) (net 12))
 (segment (start 74.972 110.61) (end 74.972 109.11) (width 0.8) (layer F.Cu) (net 16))
 (segment (start 74.972 109.11) (end 76.222 107.86) (width 0.8) (layer F.Cu) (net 16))
 (segment (start 76.222 107.86) (end 79.972 107.86) (width 0.8) (layer F.Cu) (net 16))
 (segment (start 79.972 107.86) (end 81.472 109.36) (width 0.8) (layer F.Cu) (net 16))
 (segment (start 81.472 109.36) (end 81.472 119.61) (width 0.8) (layer F.Cu) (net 16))
 (segment (start 81.472 119.61) (end 82.682 120.82) (width 0.8) (layer F.Cu) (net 16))
 (segment (start 82.682 120.82) (end 84.472 120.82) (width 0.8) (layer F.Cu) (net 16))
 (segment (start 70.472 110.61) (end 74.972 110.61) (width 0.8) (layer F.Cu) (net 16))
 (segment (start 74.972 110.61) (end 74.972 110.11) (width 0.65) (layer F.Cu) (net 16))
 (segment (start 75.012 110.57) (end 74.972 110.61) (width 0.6) (layer F.Cu) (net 16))
 (segment (start 76.472 116.61) (end 78.972 114.11) (width 0.8) (layer F.Cu) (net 17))
 (segment (start 78.972 114.11) (end 78.972 110.61) (width 0.8) (layer F.Cu) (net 17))
 (segment (start 75.012 116.61) (end 76.472 116.61) (width 0.8) (layer F.Cu) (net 17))
 (segment (start 66.972 129.36) (end 74.972 129.36) (width 0.65) (layer F.Cu) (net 17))
 (segment (start 74.972 123.11) (end 74.972 129.36) (width 0.65) (layer F.Cu) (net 17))
 (segment (start 75.012 116.61) (end 75.012 123.07) (width 0.65) (layer F.Cu) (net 17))
 (segment (start 75.012 123.07) (end 74.972 123.11) (width 0.65) (layer F.Cu) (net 17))
 (segment (start 56.222 117.61) (end 64.682 117.61) (width 0.65) (layer F.Cu) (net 2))
 (segment (start 64.682 117.61) (end 64.722 117.57) (width 0.65) (layer F.Cu) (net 2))
 (segment (start 69.472 123.11) (end 66.472 120.11) (width 0.65) (layer F.Cu) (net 4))
 (segment (start 66.472 120.11) (end 64.722 120.11) (width 0.65) (layer F.Cu) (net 4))
 (segment (start 70.972 123.11) (end 69.472 123.11) (width 0.65) (layer F.Cu) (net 4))
 (segment (start 104.472 122.36) (end 104.472 97.11) (width 0.55) (layer F.Cu) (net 15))
 (segment (start 104.472 97.11) (end 102.722 95.36) (width 0.55) (layer F.Cu) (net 15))
 (segment (start 102.722 124.11) (end 104.472 122.36) (width 0.55) (layer F.Cu) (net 15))
 (segment (start 98.222 124.11) (end 102.722 124.11) (width 0.55) (layer F.Cu) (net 15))
 (segment (start 96.972 122.86) (end 98.222 124.11) (width 0.55) (layer F.Cu) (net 15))
 (segment (start 96.972 120.86) (end 96.972 122.86) (width 0.55) (layer F.Cu) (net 15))
 (segment (start 92.092 120.82) (end 96.932 120.82) (width 0.8) (layer F.Cu) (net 15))
 (segment (start 96.932 120.82) (end 96.972 120.86) (width 0.8) (layer F.Cu) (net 15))
 (segment (start 72.972 75.61) (end 64.650932 75.61) (width 1.5) (layer F.Cu) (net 6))
 (segment (start 64.650932 75.61) (end 59.436466 80.824466) (width 1.5) (layer F.Cu) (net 6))
 (segment (start 59.436466 80.824466) (end 59.436466 99.324466) (width 1.5) (layer F.Cu) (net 6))
 (segment (start 59.436466 99.324466) (end 59.497126 99.385126) (width 1.5) (layer F.Cu) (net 6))
 (segment (start 85.472 72.11) (end 86.472 73.11) (width 1.5) (layer F.Cu) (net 6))
 (segment (start 86.472 73.11) (end 86.472 75.61) (width 1.5) (layer F.Cu) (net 6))
 (segment (start 77.972 72.11) (end 85.472 72.11) (width 1.5) (layer F.Cu) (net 6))
 (segment (start 74.472 75.61) (end 77.972 72.11) (width 1.5) (layer F.Cu) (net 6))
 (segment (start 72.972 75.61) (end 74.472 75.61) (width 1.5) (layer F.Cu) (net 6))
 (segment (start 98.472 75.61) (end 98.472 80.61) (width 0.65) (layer F.Cu) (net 20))
 (segment (start 89.012 75.61) (end 98.472 75.61) (width 1.5) (layer F.Cu) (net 20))
 (segment (start 83.972 88.86) (end 78.972 88.86) (width 0.8) (layer F.Cu) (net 11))
 (segment (start 83.972 88.86) (end 83.972 75.65) (width 0.8) (layer F.Cu) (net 11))
 (segment (start 83.972 75.65) (end 83.932 75.61) (width 0.8) (layer F.Cu) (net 11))
 (segment (start 85.972 92.86) (end 89.722 89.11) (width 0.8) (layer F.Cu) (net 21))
 (segment (start 89.722 89.11) (end 89.722 86.86) (width 0.8) (layer F.Cu) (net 21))
 (segment (start 83.972 92.86) (end 85.972 92.86) (width 0.8) (layer F.Cu) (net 21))
 (segment (start 78.972 92.86) (end 83.972 92.86) (width 0.8) (layer F.Cu) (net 21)))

